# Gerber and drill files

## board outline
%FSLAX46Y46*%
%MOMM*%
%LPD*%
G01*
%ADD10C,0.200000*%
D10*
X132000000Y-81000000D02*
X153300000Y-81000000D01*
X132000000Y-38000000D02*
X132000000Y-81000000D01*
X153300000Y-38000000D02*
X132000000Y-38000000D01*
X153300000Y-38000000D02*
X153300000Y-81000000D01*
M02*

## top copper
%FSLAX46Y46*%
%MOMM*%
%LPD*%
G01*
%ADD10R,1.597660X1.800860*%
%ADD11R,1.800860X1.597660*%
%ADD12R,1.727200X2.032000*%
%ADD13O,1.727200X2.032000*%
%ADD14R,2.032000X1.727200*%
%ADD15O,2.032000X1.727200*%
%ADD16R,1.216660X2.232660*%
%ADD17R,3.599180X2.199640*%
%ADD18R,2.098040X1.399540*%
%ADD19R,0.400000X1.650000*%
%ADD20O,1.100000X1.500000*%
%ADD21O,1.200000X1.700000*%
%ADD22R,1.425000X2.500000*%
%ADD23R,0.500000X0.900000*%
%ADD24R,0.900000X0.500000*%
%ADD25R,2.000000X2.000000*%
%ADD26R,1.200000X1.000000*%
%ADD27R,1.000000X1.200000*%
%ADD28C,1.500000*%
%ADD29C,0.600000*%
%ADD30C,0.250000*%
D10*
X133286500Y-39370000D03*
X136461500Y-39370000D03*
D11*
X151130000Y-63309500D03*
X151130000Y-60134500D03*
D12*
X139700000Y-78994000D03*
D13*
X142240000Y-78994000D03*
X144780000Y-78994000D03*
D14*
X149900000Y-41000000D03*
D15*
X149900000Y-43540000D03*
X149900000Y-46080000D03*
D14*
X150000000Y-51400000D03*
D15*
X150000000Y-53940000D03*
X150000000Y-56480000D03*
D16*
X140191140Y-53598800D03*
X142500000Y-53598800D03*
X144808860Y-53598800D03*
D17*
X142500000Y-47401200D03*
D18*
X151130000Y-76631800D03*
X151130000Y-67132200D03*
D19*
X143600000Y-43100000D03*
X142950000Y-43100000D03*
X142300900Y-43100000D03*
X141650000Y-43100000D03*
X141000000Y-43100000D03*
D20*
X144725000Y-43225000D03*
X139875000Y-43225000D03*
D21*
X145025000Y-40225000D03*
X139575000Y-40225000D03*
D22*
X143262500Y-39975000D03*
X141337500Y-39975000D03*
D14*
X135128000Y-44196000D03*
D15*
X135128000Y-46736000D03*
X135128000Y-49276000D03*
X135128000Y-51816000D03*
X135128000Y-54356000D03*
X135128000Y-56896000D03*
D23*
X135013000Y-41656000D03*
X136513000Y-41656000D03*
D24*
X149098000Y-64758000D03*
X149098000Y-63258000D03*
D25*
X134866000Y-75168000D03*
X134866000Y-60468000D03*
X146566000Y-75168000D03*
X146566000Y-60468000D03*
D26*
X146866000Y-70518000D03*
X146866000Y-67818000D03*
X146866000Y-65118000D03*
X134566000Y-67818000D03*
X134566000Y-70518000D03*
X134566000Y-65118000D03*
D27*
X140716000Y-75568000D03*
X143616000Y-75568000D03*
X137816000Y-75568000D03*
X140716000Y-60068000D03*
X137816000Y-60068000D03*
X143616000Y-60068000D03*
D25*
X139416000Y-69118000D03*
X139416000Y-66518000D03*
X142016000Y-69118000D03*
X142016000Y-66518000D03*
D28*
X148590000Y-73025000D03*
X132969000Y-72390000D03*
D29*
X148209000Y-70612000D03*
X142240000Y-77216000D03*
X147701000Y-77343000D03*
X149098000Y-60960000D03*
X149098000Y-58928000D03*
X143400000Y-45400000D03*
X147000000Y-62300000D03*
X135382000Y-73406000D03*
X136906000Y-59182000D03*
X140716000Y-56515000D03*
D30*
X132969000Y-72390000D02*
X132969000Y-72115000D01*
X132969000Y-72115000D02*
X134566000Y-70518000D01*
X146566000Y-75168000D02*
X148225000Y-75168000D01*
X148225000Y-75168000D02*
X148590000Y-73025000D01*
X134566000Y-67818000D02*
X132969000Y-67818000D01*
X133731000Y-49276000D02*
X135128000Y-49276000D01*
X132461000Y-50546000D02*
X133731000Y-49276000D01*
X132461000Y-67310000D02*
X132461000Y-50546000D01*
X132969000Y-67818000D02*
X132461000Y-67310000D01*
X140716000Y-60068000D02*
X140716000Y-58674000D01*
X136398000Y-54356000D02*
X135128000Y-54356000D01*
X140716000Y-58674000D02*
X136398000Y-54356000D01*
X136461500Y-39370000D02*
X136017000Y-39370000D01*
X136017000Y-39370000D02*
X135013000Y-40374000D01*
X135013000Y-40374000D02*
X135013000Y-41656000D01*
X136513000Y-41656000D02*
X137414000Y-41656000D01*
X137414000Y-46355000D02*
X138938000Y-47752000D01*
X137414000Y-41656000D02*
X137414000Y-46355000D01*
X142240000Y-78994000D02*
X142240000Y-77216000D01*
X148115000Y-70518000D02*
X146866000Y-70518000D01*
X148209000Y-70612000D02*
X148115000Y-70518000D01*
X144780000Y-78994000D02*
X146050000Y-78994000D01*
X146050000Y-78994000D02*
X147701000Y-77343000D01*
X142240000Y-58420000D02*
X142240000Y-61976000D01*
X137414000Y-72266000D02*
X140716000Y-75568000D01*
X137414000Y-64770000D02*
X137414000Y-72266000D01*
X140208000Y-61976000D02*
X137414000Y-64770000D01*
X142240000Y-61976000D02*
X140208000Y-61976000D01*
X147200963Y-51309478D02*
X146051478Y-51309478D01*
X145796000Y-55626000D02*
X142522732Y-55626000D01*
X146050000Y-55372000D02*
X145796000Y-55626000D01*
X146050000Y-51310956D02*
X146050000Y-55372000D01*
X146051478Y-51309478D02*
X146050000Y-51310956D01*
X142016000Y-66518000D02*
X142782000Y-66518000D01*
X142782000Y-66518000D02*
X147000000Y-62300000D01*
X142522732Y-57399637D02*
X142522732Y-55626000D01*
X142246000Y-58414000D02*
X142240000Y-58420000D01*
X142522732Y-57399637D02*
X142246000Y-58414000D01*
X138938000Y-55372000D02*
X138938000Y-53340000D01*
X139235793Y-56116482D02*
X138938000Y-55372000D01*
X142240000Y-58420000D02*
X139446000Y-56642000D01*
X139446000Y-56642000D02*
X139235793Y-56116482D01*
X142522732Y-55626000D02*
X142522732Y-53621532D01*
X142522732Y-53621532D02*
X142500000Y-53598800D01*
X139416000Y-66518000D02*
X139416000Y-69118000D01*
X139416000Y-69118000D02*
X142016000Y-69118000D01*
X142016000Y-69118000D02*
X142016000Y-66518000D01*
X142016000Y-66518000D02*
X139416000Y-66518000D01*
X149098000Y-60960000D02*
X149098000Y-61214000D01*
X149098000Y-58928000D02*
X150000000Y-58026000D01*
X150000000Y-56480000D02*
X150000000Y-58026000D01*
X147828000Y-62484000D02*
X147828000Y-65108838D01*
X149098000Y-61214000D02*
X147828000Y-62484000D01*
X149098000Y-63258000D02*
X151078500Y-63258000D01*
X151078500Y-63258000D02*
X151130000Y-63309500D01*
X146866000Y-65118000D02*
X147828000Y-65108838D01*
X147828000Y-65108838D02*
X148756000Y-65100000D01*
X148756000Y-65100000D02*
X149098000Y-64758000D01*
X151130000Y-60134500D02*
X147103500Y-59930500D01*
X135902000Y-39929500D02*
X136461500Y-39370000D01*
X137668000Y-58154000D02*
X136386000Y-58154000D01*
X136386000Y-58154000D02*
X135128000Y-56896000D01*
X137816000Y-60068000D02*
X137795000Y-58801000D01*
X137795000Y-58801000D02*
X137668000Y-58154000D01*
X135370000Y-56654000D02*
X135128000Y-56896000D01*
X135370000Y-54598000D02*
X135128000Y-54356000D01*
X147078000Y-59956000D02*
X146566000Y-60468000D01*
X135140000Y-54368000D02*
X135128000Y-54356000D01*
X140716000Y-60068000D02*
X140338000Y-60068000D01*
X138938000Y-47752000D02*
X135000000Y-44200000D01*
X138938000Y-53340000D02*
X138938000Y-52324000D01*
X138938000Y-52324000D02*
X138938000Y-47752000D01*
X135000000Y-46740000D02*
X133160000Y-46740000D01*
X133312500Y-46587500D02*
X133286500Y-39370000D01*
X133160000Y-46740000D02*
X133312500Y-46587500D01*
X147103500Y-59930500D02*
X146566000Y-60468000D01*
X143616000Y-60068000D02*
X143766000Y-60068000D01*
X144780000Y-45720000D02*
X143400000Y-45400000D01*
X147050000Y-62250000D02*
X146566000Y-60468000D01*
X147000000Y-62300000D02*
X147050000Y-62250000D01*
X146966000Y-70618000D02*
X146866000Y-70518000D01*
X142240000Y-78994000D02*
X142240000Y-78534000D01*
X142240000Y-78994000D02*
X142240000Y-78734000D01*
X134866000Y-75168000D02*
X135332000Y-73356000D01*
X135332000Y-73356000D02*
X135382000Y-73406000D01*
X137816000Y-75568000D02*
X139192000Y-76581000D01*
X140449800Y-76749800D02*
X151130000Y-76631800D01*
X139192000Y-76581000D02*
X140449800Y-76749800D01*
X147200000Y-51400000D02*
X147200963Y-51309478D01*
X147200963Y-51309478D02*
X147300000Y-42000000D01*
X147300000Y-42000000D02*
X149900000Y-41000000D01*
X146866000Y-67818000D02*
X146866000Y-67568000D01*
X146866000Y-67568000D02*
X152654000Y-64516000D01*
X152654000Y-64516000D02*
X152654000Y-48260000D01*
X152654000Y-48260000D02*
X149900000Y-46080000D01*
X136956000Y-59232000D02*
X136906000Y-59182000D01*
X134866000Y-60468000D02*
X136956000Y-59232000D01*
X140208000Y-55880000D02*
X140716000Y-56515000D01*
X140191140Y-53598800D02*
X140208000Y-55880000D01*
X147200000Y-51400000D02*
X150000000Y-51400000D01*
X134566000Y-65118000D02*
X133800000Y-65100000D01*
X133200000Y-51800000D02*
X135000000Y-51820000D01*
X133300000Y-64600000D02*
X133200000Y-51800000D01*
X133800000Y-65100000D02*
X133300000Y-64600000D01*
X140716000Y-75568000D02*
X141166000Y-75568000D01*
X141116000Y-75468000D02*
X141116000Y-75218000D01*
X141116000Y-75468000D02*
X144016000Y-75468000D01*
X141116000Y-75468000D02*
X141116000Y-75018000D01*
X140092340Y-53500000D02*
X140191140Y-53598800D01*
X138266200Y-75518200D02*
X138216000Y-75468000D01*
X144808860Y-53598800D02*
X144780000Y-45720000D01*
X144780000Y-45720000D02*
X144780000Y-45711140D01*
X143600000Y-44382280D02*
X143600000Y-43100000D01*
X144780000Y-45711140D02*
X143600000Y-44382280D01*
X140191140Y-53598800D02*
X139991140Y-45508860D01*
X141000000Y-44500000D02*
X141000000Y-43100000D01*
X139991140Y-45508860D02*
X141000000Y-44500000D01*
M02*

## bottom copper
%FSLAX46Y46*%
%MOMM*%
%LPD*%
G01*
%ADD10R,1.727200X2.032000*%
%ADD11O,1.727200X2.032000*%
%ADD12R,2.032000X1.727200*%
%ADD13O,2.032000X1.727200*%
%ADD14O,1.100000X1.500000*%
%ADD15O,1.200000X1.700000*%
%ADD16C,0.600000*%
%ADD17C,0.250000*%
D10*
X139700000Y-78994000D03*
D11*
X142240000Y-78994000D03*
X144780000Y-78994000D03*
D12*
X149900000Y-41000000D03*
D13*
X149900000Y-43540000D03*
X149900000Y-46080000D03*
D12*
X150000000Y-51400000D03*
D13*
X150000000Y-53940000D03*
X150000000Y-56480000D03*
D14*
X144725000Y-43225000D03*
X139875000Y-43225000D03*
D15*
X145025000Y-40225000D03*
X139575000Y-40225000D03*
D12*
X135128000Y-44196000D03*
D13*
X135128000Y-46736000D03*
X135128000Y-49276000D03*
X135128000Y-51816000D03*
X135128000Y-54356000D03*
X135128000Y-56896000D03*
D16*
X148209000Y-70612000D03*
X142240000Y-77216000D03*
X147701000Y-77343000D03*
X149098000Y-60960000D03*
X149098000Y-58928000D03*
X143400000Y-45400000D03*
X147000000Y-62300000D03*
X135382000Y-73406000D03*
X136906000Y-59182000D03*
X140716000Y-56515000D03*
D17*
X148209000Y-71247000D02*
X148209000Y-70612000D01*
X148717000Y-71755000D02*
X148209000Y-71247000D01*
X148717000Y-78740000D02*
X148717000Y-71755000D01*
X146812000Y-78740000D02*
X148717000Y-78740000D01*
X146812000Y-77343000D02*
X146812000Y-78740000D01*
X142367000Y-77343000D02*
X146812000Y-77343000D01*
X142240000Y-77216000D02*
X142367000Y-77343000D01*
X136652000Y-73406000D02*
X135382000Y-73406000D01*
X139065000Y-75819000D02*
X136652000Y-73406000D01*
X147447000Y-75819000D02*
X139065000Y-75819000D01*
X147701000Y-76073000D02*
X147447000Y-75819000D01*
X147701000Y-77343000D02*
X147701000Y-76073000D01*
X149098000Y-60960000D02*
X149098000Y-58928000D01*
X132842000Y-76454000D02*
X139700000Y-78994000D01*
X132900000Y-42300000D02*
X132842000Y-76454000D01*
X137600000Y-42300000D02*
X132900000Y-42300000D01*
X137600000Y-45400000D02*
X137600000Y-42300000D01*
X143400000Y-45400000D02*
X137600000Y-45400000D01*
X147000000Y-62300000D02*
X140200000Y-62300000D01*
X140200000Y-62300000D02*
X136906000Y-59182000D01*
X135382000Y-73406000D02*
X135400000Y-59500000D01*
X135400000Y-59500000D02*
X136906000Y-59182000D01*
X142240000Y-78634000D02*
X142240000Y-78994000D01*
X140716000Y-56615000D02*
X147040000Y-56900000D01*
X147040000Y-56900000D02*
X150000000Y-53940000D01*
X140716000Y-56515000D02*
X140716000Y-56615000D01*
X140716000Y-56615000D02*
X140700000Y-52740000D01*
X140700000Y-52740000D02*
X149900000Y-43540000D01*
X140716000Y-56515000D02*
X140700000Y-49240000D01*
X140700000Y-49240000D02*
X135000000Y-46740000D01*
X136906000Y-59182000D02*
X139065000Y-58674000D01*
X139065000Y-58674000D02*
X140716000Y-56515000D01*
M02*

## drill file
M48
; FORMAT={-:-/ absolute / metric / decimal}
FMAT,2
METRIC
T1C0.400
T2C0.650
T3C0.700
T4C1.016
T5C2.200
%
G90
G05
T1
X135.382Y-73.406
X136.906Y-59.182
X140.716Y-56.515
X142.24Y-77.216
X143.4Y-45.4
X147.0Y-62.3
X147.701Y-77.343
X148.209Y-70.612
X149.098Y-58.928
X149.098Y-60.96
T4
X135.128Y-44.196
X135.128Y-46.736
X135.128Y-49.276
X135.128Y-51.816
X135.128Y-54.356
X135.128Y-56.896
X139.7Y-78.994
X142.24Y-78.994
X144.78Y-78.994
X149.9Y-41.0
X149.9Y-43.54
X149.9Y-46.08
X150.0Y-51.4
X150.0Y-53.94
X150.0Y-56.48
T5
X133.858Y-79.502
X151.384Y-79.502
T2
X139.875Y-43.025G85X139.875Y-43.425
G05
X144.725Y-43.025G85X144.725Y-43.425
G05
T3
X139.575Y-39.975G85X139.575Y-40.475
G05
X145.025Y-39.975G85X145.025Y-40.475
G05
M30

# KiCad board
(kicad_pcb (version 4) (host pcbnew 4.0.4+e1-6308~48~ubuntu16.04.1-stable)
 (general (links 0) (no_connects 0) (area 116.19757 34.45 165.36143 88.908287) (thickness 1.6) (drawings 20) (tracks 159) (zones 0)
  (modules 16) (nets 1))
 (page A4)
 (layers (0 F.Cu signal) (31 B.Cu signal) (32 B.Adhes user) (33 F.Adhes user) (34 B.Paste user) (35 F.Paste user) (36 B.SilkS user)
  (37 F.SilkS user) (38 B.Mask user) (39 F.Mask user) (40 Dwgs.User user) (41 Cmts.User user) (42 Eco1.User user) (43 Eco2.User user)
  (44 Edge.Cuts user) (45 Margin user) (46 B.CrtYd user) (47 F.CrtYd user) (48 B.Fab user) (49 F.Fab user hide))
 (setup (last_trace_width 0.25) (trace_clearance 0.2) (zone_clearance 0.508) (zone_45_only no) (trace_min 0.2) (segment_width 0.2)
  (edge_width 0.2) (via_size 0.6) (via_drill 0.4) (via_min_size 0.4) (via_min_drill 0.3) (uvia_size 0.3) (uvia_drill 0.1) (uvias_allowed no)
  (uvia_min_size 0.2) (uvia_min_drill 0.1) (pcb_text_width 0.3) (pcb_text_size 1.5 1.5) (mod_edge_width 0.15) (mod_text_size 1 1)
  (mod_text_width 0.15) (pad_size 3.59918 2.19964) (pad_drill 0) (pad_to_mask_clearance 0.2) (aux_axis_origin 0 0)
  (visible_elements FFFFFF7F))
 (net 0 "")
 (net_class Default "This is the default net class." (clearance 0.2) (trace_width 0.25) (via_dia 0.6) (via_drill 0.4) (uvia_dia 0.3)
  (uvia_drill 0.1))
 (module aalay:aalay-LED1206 (layer F.Cu) (at 134.874 39.37)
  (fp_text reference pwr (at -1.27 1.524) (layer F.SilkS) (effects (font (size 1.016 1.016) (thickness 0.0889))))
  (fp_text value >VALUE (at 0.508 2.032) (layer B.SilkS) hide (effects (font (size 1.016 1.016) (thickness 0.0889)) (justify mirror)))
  (pad A smd rect (at -1.5875 0) (size 1.59766 1.80086) (layers F.Cu F.Paste F.Mask))
  (pad K smd rect (at 1.5875 0) (size 1.59766 1.80086) (layers F.Cu F.Paste F.Mask)))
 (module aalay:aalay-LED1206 (layer F.Cu) (at 151.13 61.722 90)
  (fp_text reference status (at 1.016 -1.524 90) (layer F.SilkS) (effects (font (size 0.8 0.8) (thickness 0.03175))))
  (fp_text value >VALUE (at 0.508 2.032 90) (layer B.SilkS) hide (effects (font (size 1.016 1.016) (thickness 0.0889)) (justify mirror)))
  (pad A smd rect (at -1.5875 0 90) (size 1.59766 1.80086) (layers F.Cu F.Paste F.Mask))
  (pad K smd rect (at 1.5875 0 90) (size 1.59766 1.80086) (layers F.Cu F.Paste F.Mask)))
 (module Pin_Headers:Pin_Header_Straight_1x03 (layer F.Cu) (at 139.7 78.994 90)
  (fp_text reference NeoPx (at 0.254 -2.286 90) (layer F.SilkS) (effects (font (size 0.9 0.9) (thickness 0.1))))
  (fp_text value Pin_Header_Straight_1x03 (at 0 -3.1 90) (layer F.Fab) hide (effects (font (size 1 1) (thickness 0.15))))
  (pad 1 thru_hole rect (at 0 0 90) (size 2.032 1.7272) (drill 1.016) (layers *.Cu *.Mask F.SilkS))
  (pad 2 thru_hole oval (at 0 2.54 90) (size 2.032 1.7272) (drill 1.016) (layers *.Cu *.Mask F.SilkS))
  (pad 3 thru_hole oval (at 0 5.08 90) (size 2.032 1.7272) (drill 1.016) (layers *.Cu *.Mask F.SilkS)))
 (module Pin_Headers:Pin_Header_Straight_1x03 (layer F.Cu) (at 149.9 41)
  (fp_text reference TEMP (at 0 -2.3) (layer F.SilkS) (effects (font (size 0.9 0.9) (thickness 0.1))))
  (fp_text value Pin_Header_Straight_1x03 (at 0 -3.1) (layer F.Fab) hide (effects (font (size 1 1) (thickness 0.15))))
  (pad 1 thru_hole rect (at 0 0) (size 2.032 1.7272) (drill 1.016) (layers *.Cu *.Mask F.SilkS))
  (pad 2 thru_hole oval (at 0 2.54) (size 2.032 1.7272) (drill 1.016) (layers *.Cu *.Mask F.SilkS))
  (pad 3 thru_hole oval (at 0 5.08) (size 2.032 1.7272) (drill 1.016) (layers *.Cu *.Mask F.SilkS)))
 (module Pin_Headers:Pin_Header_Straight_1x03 (layer F.Cu) (at 150 51.4)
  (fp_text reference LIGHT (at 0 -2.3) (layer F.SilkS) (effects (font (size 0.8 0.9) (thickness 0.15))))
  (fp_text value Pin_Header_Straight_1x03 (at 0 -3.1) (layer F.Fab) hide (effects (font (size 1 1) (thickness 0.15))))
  (pad 1 thru_hole rect (at 0 0) (size 2.032 1.7272) (drill 1.016) (layers *.Cu *.Mask F.SilkS))
  (pad 2 thru_hole oval (at 0 2.54) (size 2.032 1.7272) (drill 1.016) (layers *.Cu *.Mask F.SilkS))
  (pad 3 thru_hole oval (at 0 5.08) (size 2.032 1.7272) (drill 1.016) (layers *.Cu *.Mask F.SilkS)))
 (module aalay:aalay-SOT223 (layer F.Cu) (at 142.5 50.5)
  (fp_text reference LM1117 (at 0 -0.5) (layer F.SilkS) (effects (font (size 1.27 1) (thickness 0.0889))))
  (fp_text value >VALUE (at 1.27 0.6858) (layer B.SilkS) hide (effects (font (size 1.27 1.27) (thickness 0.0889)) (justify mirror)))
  (pad GND smd rect (at -2.30886 3.0988) (size 1.21666 2.23266) (layers F.Cu F.Paste F.Mask))
  (pad OUT smd rect (at 0 3.0988) (size 1.21666 2.23266) (layers F.Cu F.Paste F.Mask))
  (pad IN smd rect (at 2.30886 3.0988) (size 1.21666 2.23266) (layers F.Cu F.Paste F.Mask))
  (pad OUT smd rect (at 0 -3.0988) (size 3.59918 2.19964) (layers F.Cu F.Paste F.Mask)))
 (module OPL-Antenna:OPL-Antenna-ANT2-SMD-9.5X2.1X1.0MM (layer F.Cu) (at 151.13 71.882 90)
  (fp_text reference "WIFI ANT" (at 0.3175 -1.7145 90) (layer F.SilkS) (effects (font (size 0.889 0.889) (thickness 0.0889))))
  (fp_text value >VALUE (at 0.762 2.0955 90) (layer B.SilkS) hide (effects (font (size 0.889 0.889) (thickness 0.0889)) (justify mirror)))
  (pad 1 smd rect (at -4.7498 0 90) (size 1.39954 2.09804) (layers F.Cu F.Paste F.Mask))
  (pad 2 smd rect (at 4.7498 0 90) (size 1.39954 2.09804) (layers F.Cu F.Paste F.Mask)))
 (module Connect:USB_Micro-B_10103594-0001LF (layer F.Cu) (at 142.3 41.6 180)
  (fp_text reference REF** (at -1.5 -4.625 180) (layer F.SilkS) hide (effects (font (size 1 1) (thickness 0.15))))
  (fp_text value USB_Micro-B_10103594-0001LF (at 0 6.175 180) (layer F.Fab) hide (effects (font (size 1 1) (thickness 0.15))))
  (pad +5 smd rect (at -1.3 -1.5 270) (size 1.65 0.4) (layers F.Cu F.Paste F.Mask))
  (pad D- smd rect (at -0.65 -1.5 270) (size 1.65 0.4) (layers F.Cu F.Paste F.Mask))
  (pad D+ smd rect (at -0.0009 -1.5 270) (size 1.65 0.4) (layers F.Cu F.Paste F.Mask))
  (pad ID smd rect (at 0.65 -1.5 270) (size 1.65 0.4) (layers F.Cu F.Paste F.Mask))
  (pad GND smd rect (at 1.3 -1.5 270) (size 1.65 0.4) (layers F.Cu F.Paste F.Mask))
  (pad 6 thru_hole oval (at -2.425 -1.625 270) (size 1.5 1.1) (drill oval 1.05 0.65) (layers *.Cu *.Mask F.SilkS))
  (pad 6 thru_hole oval (at 2.425 -1.625 270) (size 1.5 1.1) (drill oval 1.05 0.65) (layers *.Cu *.Mask F.SilkS))
  (pad 6 thru_hole oval (at -2.725 1.375 270) (size 1.7 1.2) (drill oval 1.2 0.7) (layers *.Cu *.Mask F.SilkS))
  (pad 6 thru_hole oval (at 2.725 1.375 270) (size 1.7 1.2) (drill oval 1.2 0.7) (layers *.Cu *.Mask F.SilkS))
  (pad 6 smd rect (at -0.9625 1.625 270) (size 2.5 1.425) (layers F.Cu F.Paste F.Mask))
  (pad 6 smd rect (at 0.9625 1.625 270) (size 2.5 1.425) (layers F.Cu F.Paste F.Mask)))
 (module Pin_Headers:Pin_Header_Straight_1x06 (layer F.Cu) (at 135.128 44.196)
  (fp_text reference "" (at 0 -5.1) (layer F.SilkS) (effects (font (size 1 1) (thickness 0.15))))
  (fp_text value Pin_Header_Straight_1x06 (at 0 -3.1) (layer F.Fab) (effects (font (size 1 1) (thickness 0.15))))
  (pad 1 thru_hole rect (at 0 0) (size 2.032 1.7272) (drill 1.016) (layers *.Cu *.Mask F.SilkS))
  (pad 2 thru_hole oval (at 0 2.54) (size 2.032 1.7272) (drill 1.016) (layers *.Cu *.Mask F.SilkS))
  (pad 3 thru_hole oval (at 0 5.08) (size 2.032 1.7272) (drill 1.016) (layers *.Cu *.Mask F.SilkS))
  (pad 4 thru_hole oval (at 0 7.62) (size 2.032 1.7272) (drill 1.016) (layers *.Cu *.Mask F.SilkS))
  (pad 5 thru_hole oval (at 0 10.16) (size 2.032 1.7272) (drill 1.016) (layers *.Cu *.Mask F.SilkS))
  (pad 6 thru_hole oval (at 0 12.7) (size 2.032 1.7272) (drill 1.016) (layers *.Cu *.Mask F.SilkS)))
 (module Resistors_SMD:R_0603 (layer F.Cu) (at 135.763 41.656)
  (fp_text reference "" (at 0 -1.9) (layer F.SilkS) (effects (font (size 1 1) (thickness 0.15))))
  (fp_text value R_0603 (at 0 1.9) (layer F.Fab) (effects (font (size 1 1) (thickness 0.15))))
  (pad 1 smd rect (at -0.75 0) (size 0.5 0.9) (layers F.Cu F.Paste F.Mask))
  (pad 2 smd rect (at 0.75 0) (size 0.5 0.9) (layers F.Cu F.Paste F.Mask)))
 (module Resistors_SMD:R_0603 (layer F.Cu) (at 149.098 64.008 90)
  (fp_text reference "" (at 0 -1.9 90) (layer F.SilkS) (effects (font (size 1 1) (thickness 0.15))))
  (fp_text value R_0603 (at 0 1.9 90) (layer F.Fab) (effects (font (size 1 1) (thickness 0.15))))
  (pad 1 smd rect (at -0.75 0 90) (size 0.5 0.9) (layers F.Cu F.Paste F.Mask))
  (pad 2 smd rect (at 0.75 0 90) (size 0.5 0.9) (layers F.Cu F.Paste F.Mask)))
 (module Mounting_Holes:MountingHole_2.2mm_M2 (layer F.Cu) (at 133.858 79.502)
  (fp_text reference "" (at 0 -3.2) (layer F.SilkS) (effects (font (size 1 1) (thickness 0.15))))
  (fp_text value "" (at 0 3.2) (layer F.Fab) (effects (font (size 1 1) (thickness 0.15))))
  (pad 1 np_thru_hole circle (at 0 0) (size 2.2 2.2) (drill 2.2) (layers *.Cu *.Mask F.SilkS)))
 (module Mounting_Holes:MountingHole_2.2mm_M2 (layer F.Cu) (at 151.384 79.502)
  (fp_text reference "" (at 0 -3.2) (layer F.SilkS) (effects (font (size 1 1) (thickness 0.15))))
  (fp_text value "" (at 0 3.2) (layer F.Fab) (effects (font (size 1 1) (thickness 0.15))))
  (pad 1 np_thru_hole circle (at 0 0) (size 2.2 2.2) (drill 2.2) (layers *.Cu *.Mask F.SilkS)))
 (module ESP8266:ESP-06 (layer F.Cu) (at 140.716 67.818 90)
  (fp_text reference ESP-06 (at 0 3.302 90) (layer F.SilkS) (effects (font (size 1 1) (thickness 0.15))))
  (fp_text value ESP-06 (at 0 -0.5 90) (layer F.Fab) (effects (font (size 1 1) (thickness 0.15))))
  (pad GND smd rect (at -7.35 -5.85 90) (size 2 2) (layers F.Cu F.Paste F.Mask))
  (pad GP5 smd rect (at 7.35 -5.85 90) (size 2 2) (layers F.Cu F.Paste F.Mask))
  (pad GP16 smd rect (at -7.35 5.85 90) (size 2 2) (layers F.Cu F.Paste F.Mask))
  (pad GP15 smd rect (at 7.35 5.85 90) (size 2 2) (layers F.Cu F.Paste F.Mask))
  (pad GP14 smd rect (at -2.7 6.15 90) (size 1 1.2) (layers F.Cu F.Paste F.Mask))
  (pad GP12 smd rect (at 0 6.15 90) (size 1 1.2) (layers F.Cu F.Paste F.Mask))
  (pad GP13 smd rect (at 2.7 6.15 90) (size 1 1.2) (layers F.Cu F.Paste F.Mask))
  (pad TX smd rect (at 0 -6.15 90) (size 1 1.2) (layers F.Cu F.Paste F.Mask))
  (pad RST smd rect (at -2.7 -6.15 90) (size 1 1.2) (layers F.Cu F.Paste F.Mask))
  (pad RX smd rect (at 2.7 -6.15 90) (size 1 1.2) (layers F.Cu F.Paste F.Mask))
  (pad 3.3 smd rect (at -7.75 0 90) (size 1.2 1) (layers F.Cu F.Paste F.Mask))
  (pad CHPD smd rect (at -7.75 2.9 90) (size 1.2 1) (layers F.Cu F.Paste F.Mask))
  (pad ANT smd rect (at -7.75 -2.9 90) (size 1.2 1) (layers F.Cu F.Paste F.Mask))
  (pad GP2 smd rect (at 7.75 0 90) (size 1.2 1) (layers F.Cu F.Paste F.Mask))
  (pad GP0 smd rect (at 7.75 -2.9 90) (size 1.2 1) (layers F.Cu F.Paste F.Mask))
  (pad GP4 smd rect (at 7.75 2.9 90) (size 1.2 1) (layers F.Cu F.Paste F.Mask))
  (pad GND smd rect (at -1.3 -1.3 90) (size 2 2) (layers F.Cu F.Paste F.Mask))
  (pad GND smd rect (at 1.3 -1.3 90) (size 2 2) (layers F.Cu F.Paste F.Mask))
  (pad GND smd rect (at -1.3 1.3 90) (size 2 2) (layers F.Cu F.Paste F.Mask))
  (pad GND smd rect (at 1.3 1.3 90) (size 2 2) (layers F.Cu F.Paste F.Mask)))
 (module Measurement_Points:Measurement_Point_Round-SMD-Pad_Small (layer F.Cu) (at 148.59 73.025)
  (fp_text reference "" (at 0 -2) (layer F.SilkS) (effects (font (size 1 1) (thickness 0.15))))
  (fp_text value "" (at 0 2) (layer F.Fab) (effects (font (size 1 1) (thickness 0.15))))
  (pad 1 smd circle (at 0 0) (size 1.5 1.5) (layers F.Cu F.Mask)))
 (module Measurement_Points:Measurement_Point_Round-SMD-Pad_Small (layer F.Cu) (at 132.969 72.39)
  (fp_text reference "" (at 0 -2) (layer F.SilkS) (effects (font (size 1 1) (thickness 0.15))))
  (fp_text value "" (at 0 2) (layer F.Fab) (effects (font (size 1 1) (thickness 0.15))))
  (pad 1 smd circle (at 0 0) (size 1.5 1.5) (layers F.Cu F.Mask)))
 (gr_line (start 132 81) (end 153.3 81) (angle 90) (layer Edge.Cuts) (width 0.2))
 (gr_line (start 132 38) (end 132 81) (angle 90) (layer Edge.Cuts) (width 0.2))
 (gr_line (start 153.3 38) (end 132 38) (angle 90) (layer Edge.Cuts) (width 0.2))
 (gr_line (start 153.3 38) (end 153.3 81) (angle 90) (layer Edge.Cuts) (width 0.2))
 (segment (start 132.969 72.39) (end 132.969 72.115) (width 0.25) (layer F.Cu) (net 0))
 (segment (start 132.969 72.115) (end 134.566 70.518) (width 0.25) (layer F.Cu) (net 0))
 (segment (start 146.566 75.168) (end 148.225 75.168) (width 0.25) (layer F.Cu) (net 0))
 (segment (start 148.225 75.168) (end 148.59 73.025) (width 0.25) (layer F.Cu) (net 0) (status 20))
 (segment (start 134.566 67.818) (end 132.969 67.818) (width 0.25) (layer F.Cu) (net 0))
 (segment (start 133.731 49.276) (end 135.128 49.276) (width 0.25) (layer F.Cu) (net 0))
 (segment (start 132.461 50.546) (end 133.731 49.276) (width 0.25) (layer F.Cu) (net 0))
 (segment (start 132.461 67.31) (end 132.461 50.546) (width 0.25) (layer F.Cu) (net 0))
 (segment (start 132.969 67.818) (end 132.461 67.31) (width 0.25) (layer F.Cu) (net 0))
 (segment (start 140.716 60.068) (end 140.716 58.674) (width 0.25) (layer F.Cu) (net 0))
 (segment (start 136.398 54.356) (end 135.128 54.356) (width 0.25) (layer F.Cu) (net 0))
 (segment (start 140.716 58.674) (end 136.398 54.356) (width 0.25) (layer F.Cu) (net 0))
 (segment (start 136.4615 39.37) (end 136.017 39.37) (width 0.25) (layer F.Cu) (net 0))
 (segment (start 136.017 39.37) (end 135.013 40.374) (width 0.25) (layer F.Cu) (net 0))
 (segment (start 135.013 40.374) (end 135.013 41.656) (width 0.25) (layer F.Cu) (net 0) (status 20))
 (segment (start 136.513 41.656) (end 137.414 41.656) (width 0.25) (layer F.Cu) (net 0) (status 10))
 (segment (start 137.414 46.355) (end 138.938 47.752) (width 0.25) (layer F.Cu) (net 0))
 (segment (start 137.414 41.656) (end 137.414 46.355) (width 0.25) (layer F.Cu) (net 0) (status 10))
 (segment (start 142.24 78.994) (end 142.24 77.216) (width 0.25) (layer F.Cu) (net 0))
 (segment (start 148.115 70.518) (end 146.866 70.518) (width 0.25) (layer F.Cu) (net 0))
 (segment (start 148.209 70.612) (end 148.115 70.518) (width 0.25) (layer F.Cu) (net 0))
 (via (at 148.209 70.612) (size 0.6) (drill 0.4) (layers F.Cu B.Cu) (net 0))
 (segment (start 148.209 71.247) (end 148.209 70.612) (width 0.25) (layer B.Cu) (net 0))
 (segment (start 148.717 71.755) (end 148.209 71.247) (width 0.25) (layer B.Cu) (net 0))
 (segment (start 148.717 78.74) (end 148.717 71.755) (width 0.25) (layer B.Cu) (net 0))
 (segment (start 146.812 78.74) (end 148.717 78.74) (width 0.25) (layer B.Cu) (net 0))
 (segment (start 146.812 77.343) (end 146.812 78.74) (width 0.25) (layer B.Cu) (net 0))
 (segment (start 142.367 77.343) (end 146.812 77.343) (width 0.25) (layer B.Cu) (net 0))
 (segment (start 142.24 77.216) (end 142.367 77.343) (width 0.25) (layer B.Cu) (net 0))
 (via (at 142.24 77.216) (size 0.6) (drill 0.4) (layers F.Cu B.Cu) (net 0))
 (segment (start 144.78 78.994) (end 146.05 78.994) (width 0.25) (layer F.Cu) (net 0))
 (segment (start 136.652 73.406) (end 135.382 73.406) (width 0.25) (layer B.Cu) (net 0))
 (segment (start 139.065 75.819) (end 136.652 73.406) (width 0.25) (layer B.Cu) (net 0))
 (segment (start 147.447 75.819) (end 139.065 75.819) (width 0.25) (layer B.Cu) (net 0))
 (segment (start 147.701 76.073) (end 147.447 75.819) (width 0.25) (layer B.Cu) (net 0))
 (segment (start 147.701 77.343) (end 147.701 76.073) (width 0.25) (layer B.Cu) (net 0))
 (via (at 147.701 77.343) (size 0.6) (drill 0.4) (layers F.Cu B.Cu) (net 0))
 (segment (start 146.05 78.994) (end 147.701 77.343) (width 0.25) (layer F.Cu) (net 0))
 (segment (start 142.24 58.42) (end 142.24 61.976) (width 0.25) (layer F.Cu) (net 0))
 (segment (start 137.414 72.266) (end 140.716 75.568) (width 0.25) (layer F.Cu) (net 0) (status 20))
 (segment (start 137.414 64.77) (end 137.414 72.266) (width 0.25) (layer F.Cu) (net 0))
 (segment (start 140.208 61.976) (end 137.414 64.77) (width 0.25) (layer F.Cu) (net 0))
 (segment (start 142.24 61.976) (end 140.208 61.976) (width 0.25) (layer F.Cu) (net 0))
 (segment (start 147.200963 51.309478) (end 146.051478 51.309478) (width 0.25) (layer F.Cu) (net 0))
 (segment (start 145.796 55.626) (end 142.522732 55.626) (width 0.25) (layer F.Cu) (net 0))
 (segment (start 146.05 55.372) (end 145.796 55.626) (width 0.25) (layer F.Cu) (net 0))
 (segment (start 146.05 51.310956) (end 146.05 55.372) (width 0.25) (layer F.Cu) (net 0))
 (segment (start 146.051478 51.309478) (end 146.05 51.310956) (width 0.25) (layer F.Cu) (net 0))
 (segment (start 142.016 66.518) (end 142.782 66.518) (width 0.25) (layer F.Cu) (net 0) (status 30))
 (segment (start 142.782 66.518) (end 147 62.3) (width 0.25) (layer F.Cu) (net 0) (status 10))
 (segment (start 142.522732 57.399637) (end 142.522732 55.626) (width 0.25) (layer F.Cu) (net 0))
 (segment (start 142.246 58.414) (end 142.24 58.42) (width 0.25) (layer F.Cu) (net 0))
 (segment (start 142.522732 57.399637) (end 142.246 58.414) (width 0.25) (layer F.Cu) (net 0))
 (segment (start 138.938 55.372) (end 138.938 53.34) (width 0.25) (layer F.Cu) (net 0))
 (segment (start 139.235793 56.116482) (end 138.938 55.372) (width 0.25) (layer F.Cu) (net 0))
 (segment (start 142.24 58.42) (end 139.446 56.642) (width 0.25) (layer F.Cu) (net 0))
 (segment (start 139.446 56.642) (end 139.235793 56.116482) (width 0.25) (layer F.Cu) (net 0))
 (segment (start 142.522732 55.626) (end 142.522732 53.621532) (width 0.25) (layer F.Cu) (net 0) (status 20))
 (segment (start 142.522732 53.621532) (end 142.5 53.5988) (width 0.25) (layer F.Cu) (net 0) (status 30))
 (segment (start 139.416 66.518) (end 139.416 69.118) (width 0.25) (layer F.Cu) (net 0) (status 30))
 (segment (start 139.416 69.118) (end 142.016 69.118) (width 0.25) (layer F.Cu) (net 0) (status 30))
 (segment (start 142.016 69.118) (end 142.016 66.518) (width 0.25) (layer F.Cu) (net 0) (status 30))
 (segment (start 142.016 66.518) (end 139.416 66.518) (width 0.25) (layer F.Cu) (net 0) (status 30))
 (segment (start 149.098 60.96) (end 149.098 61.214) (width 0.25) (layer F.Cu) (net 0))
 (via (at 149.098 60.96) (size 0.6) (drill 0.4) (layers F.Cu B.Cu) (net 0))
 (segment (start 149.098 60.96) (end 149.098 58.928) (width 0.25) (layer B.Cu) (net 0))
 (via (at 149.098 58.928) (size 0.6) (drill 0.4) (layers F.Cu B.Cu) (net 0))
 (segment (start 149.098 58.928) (end 150 58.026) (width 0.25) (layer F.Cu) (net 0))
 (segment (start 150 56.48) (end 150 58.026) (width 0.25) (layer F.Cu) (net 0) (status 10))
 (segment (start 147.828 62.484) (end 147.828 65.108838) (width 0.25) (layer F.Cu) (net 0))
 (segment (start 149.098 61.214) (end 147.828 62.484) (width 0.25) (layer F.Cu) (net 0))
 (segment (start 149.098 63.258) (end 151.0785 63.258) (width 0.25) (layer F.Cu) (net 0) (status 30))
 (segment (start 151.0785 63.258) (end 151.13 63.3095) (width 0.25) (layer F.Cu) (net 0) (status 30))
 (segment (start 146.866 65.118) (end 147.828 65.108838) (width 0.25) (layer F.Cu) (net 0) (status 10))
 (segment (start 147.828 65.108838) (end 148.756 65.1) (width 0.25) (layer F.Cu) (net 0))
 (segment (start 148.756 65.1) (end 149.098 64.758) (width 0.25) (layer F.Cu) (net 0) (status 20))
 (segment (start 151.13 60.1345) (end 147.1035 59.9305) (width 0.25) (layer F.Cu) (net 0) (status 30))
 (segment (start 135.902 39.9295) (end 136.4615 39.37) (width 0.25) (layer F.Cu) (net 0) (status 30))
 (segment (start 137.668 58.154) (end 136.386 58.154) (width 0.25) (layer F.Cu) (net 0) (status 10))
 (segment (start 136.386 58.154) (end 135.128 56.896) (width 0.25) (layer F.Cu) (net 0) (status 20))
 (segment (start 137.816 60.068) (end 137.795 58.801) (width 0.25) (layer F.Cu) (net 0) (status 10))
 (segment (start 137.795 58.801) (end 137.668 58.154) (width 0.25) (layer F.Cu) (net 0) (status 20))
 (segment (start 135.37 56.654) (end 135.128 56.896) (width 0.25) (layer F.Cu) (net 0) (status 30))
 (segment (start 135.37 54.598) (end 135.128 54.356) (width 0.25) (layer F.Cu) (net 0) (status 30))
 (segment (start 147.078 59.956) (end 146.566 60.468) (width 0.25) (layer F.Cu) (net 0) (status 30))
 (segment (start 135.14 54.368) (end 135.128 54.356) (width 0.25) (layer F.Cu) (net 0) (status 30))
 (segment (start 140.716 60.068) (end 140.338 60.068) (width 0.25) (layer F.Cu) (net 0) (status 30))
 (segment (start 138.938 47.752) (end 135 44.2) (width 0.25) (layer F.Cu) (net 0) (status 20))
 (segment (start 138.938 53.34) (end 138.938 52.324) (width 0.25) (layer F.Cu) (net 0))
 (segment (start 138.938 52.324) (end 138.938 47.752) (width 0.25) (layer F.Cu) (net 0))
 (segment (start 135 46.74) (end 133.16 46.74) (width 0.25) (layer F.Cu) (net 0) (status 10))
 (segment (start 133.3125 46.5875) (end 133.2865 39.37) (width 0.25) (layer F.Cu) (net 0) (status 20))
 (segment (start 133.16 46.74) (end 133.3125 46.5875) (width 0.25) (layer F.Cu) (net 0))
 (segment (start 147.1035 59.9305) (end 146.566 60.468) (width 0.25) (layer F.Cu) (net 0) (status 30))
 (segment (start 143.616 60.068) (end 143.766 60.068) (width 0.25) (layer F.Cu) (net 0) (status 30))
 (segment (start 144.78 45.72) (end 143.4 45.4) (width 0.25) (layer F.Cu) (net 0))
 (segment (start 132.842 76.454) (end 139.7 78.994) (width 0.25) (layer B.Cu) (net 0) (status 20))
 (segment (start 132.9 42.3) (end 132.842 76.454) (width 0.25) (layer B.Cu) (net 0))
 (segment (start 137.6 42.3) (end 132.9 42.3) (width 0.25) (layer B.Cu) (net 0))
 (segment (start 137.6 45.4) (end 137.6 42.3) (width 0.25) (layer B.Cu) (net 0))
 (segment (start 143.4 45.4) (end 137.6 45.4) (width 0.25) (layer B.Cu) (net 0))
 (via (at 143.4 45.4) (size 0.6) (drill 0.4) (layers F.Cu B.Cu) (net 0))
 (segment (start 147 62.3) (end 140.2 62.3) (width 0.25) (layer B.Cu) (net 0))
 (segment (start 140.2 62.3) (end 136.906 59.182) (width 0.25) (layer B.Cu) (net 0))
 (segment (start 147.05 62.25) (end 146.566 60.468) (width 0.25) (layer F.Cu) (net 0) (status 20))
 (via (at 147 62.3) (size 0.6) (drill 0.4) (layers F.Cu B.Cu) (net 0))
 (segment (start 147 62.3) (end 147.05 62.25) (width 0.25) (layer F.Cu) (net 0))
 (segment (start 146.966 70.618) (end 146.866 70.518) (width 0.25) (layer F.Cu) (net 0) (status 30))
 (segment (start 142.24 78.994) (end 142.24 78.534) (width 0.25) (layer F.Cu) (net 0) (status 30))
 (segment (start 142.24 78.994) (end 142.24 78.734) (width 0.25) (layer F.Cu) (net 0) (status 30))
 (segment (start 135.382 73.406) (end 135.4 59.5) (width 0.25) (layer B.Cu) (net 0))
 (via (at 135.382 73.406) (size 0.6) (drill 0.4) (layers F.Cu B.Cu) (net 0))
 (segment (start 134.866 75.168) (end 135.332 73.356) (width 0.25) (layer F.Cu) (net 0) (status 10))
 (segment (start 135.332 73.356) (end 135.382 73.406) (width 0.25) (layer F.Cu) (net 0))
 (segment (start 135.4 59.5) (end 136.906 59.182) (width 0.25) (layer B.Cu) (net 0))
 (segment (start 142.24 78.634) (end 142.24 78.994) (width 0.25) (layer B.Cu) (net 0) (status 30))
 (segment (start 137.816 75.568) (end 139.192 76.581) (width 0.25) (layer F.Cu) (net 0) (status 10))
 (segment (start 140.4498 76.7498) (end 151.13 76.6318) (width 0.25) (layer F.Cu) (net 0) (status 20))
 (segment (start 139.192 76.581) (end 140.4498 76.7498) (width 0.25) (layer F.Cu) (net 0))
 (segment (start 147.2 51.4) (end 147.200963 51.309478) (width 0.25) (layer F.Cu) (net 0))
 (segment (start 147.200963 51.309478) (end 147.3 42) (width 0.25) (layer F.Cu) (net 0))
 (segment (start 147.3 42) (end 149.9 41) (width 0.25) (layer F.Cu) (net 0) (status 20))
 (segment (start 140.716 56.615) (end 147.04 56.9) (width 0.25) (layer B.Cu) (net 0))
 (segment (start 147.04 56.9) (end 150 53.94) (width 0.25) (layer B.Cu) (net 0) (status 20))
 (segment (start 146.866 67.818) (end 146.866 67.568) (width 0.25) (layer F.Cu) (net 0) (status 30))
 (segment (start 146.866 67.568) (end 152.654 64.516) (width 0.25) (layer F.Cu) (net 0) (status 10))
 (segment (start 152.654 64.516) (end 152.654 48.26) (width 0.25) (layer F.Cu) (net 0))
 (segment (start 152.654 48.26) (end 149.9 46.08) (width 0.25) (layer F.Cu) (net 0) (status 20))
 (segment (start 140.716 56.515) (end 140.716 56.615) (width 0.25) (layer B.Cu) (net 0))
 (segment (start 140.716 56.615) (end 140.7 52.74) (width 0.25) (layer B.Cu) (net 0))
 (segment (start 140.7 52.74) (end 149.9 43.54) (width 0.25) (layer B.Cu) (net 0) (status 20))
 (segment (start 140.716 56.515) (end 140.7 49.24) (width 0.25) (layer B.Cu) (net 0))
 (segment (start 140.7 49.24) (end 135 46.74) (width 0.25) (layer B.Cu) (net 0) (status 20))
 (segment (start 136.906 59.182) (end 139.065 58.674) (width 0.25) (layer B.Cu) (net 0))
 (segment (start 139.065 58.674) (end 140.716 56.515) (width 0.25) (layer B.Cu) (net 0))
 (segment (start 136.956 59.232) (end 136.906 59.182) (width 0.25) (layer F.Cu) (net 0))
 (via (at 136.906 59.182) (size 0.6) (drill 0.4) (layers F.Cu B.Cu) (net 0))
 (segment (start 134.866 60.468) (end 136.956 59.232) (width 0.25) (layer F.Cu) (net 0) (status 10))
 (segment (start 140.208 55.88) (end 140.716 56.515) (width 0.25) (layer F.Cu) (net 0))
 (via (at 140.716 56.515) (size 0.6) (drill 0.4) (layers F.Cu B.Cu) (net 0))
 (segment (start 140.19114 53.5988) (end 140.208 55.88) (width 0.25) (layer F.Cu) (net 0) (status 10))
 (segment (start 147.2 51.4) (end 150 51.4) (width 0.25) (layer F.Cu) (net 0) (status 20))
 (segment (start 134.566 65.118) (end 133.8 65.1) (width 0.25) (layer F.Cu) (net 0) (status 10))
 (segment (start 133.2 51.8) (end 135 51.82) (width 0.25) (layer F.Cu) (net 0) (status 20))
 (segment (start 133.3 64.6) (end 133.2 51.8) (width 0.25) (layer F.Cu) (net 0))
 (segment (start 133.8 65.1) (end 133.3 64.6) (width 0.25) (layer F.Cu) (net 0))
 (segment (start 140.716 75.568) (end 141.166 75.568) (width 0.25) (layer F.Cu) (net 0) (status 30))
 (segment (start 141.116 75.468) (end 141.116 75.218) (width 0.25) (layer F.Cu) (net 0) (status 30))
 (segment (start 141.116 75.468) (end 144.016 75.468) (width 0.25) (layer F.Cu) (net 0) (status 30))
 (segment (start 141.116 75.468) (end 141.116 75.018) (width 0.25) (layer F.Cu) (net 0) (status 30))
 (segment (start 140.09234 53.5) (end 140.19114 53.5988) (width 0.25) (layer F.Cu) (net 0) (status 30))
 (segment (start 138.2662 75.5182) (end 138.216 75.468) (width 0.25) (layer F.Cu) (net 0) (status 30))
 (segment (start 144.80886 53.5988) (end 144.78 45.72) (width 0.25) (layer F.Cu) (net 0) (status 10))
 (segment (start 144.78 45.72) (end 144.78 45.71114) (width 0.25) (layer F.Cu) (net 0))
 (segment (start 143.6 44.38228) (end 143.6 43.1) (width 0.25) (layer F.Cu) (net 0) (status 20))
 (segment (start 144.78 45.71114) (end 143.6 44.38228) (width 0.25) (layer F.Cu) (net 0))
 (segment (start 140.19114 53.5988) (end 139.99114 45.50886) (width 0.25) (layer F.Cu) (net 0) (status 10))
 (segment (start 141 44.5) (end 141 43.1) (width 0.25) (layer F.Cu) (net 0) (status 20))
 (segment (start 139.99114 45.50886) (end 141 44.5) (width 0.25) (layer F.Cu) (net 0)))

